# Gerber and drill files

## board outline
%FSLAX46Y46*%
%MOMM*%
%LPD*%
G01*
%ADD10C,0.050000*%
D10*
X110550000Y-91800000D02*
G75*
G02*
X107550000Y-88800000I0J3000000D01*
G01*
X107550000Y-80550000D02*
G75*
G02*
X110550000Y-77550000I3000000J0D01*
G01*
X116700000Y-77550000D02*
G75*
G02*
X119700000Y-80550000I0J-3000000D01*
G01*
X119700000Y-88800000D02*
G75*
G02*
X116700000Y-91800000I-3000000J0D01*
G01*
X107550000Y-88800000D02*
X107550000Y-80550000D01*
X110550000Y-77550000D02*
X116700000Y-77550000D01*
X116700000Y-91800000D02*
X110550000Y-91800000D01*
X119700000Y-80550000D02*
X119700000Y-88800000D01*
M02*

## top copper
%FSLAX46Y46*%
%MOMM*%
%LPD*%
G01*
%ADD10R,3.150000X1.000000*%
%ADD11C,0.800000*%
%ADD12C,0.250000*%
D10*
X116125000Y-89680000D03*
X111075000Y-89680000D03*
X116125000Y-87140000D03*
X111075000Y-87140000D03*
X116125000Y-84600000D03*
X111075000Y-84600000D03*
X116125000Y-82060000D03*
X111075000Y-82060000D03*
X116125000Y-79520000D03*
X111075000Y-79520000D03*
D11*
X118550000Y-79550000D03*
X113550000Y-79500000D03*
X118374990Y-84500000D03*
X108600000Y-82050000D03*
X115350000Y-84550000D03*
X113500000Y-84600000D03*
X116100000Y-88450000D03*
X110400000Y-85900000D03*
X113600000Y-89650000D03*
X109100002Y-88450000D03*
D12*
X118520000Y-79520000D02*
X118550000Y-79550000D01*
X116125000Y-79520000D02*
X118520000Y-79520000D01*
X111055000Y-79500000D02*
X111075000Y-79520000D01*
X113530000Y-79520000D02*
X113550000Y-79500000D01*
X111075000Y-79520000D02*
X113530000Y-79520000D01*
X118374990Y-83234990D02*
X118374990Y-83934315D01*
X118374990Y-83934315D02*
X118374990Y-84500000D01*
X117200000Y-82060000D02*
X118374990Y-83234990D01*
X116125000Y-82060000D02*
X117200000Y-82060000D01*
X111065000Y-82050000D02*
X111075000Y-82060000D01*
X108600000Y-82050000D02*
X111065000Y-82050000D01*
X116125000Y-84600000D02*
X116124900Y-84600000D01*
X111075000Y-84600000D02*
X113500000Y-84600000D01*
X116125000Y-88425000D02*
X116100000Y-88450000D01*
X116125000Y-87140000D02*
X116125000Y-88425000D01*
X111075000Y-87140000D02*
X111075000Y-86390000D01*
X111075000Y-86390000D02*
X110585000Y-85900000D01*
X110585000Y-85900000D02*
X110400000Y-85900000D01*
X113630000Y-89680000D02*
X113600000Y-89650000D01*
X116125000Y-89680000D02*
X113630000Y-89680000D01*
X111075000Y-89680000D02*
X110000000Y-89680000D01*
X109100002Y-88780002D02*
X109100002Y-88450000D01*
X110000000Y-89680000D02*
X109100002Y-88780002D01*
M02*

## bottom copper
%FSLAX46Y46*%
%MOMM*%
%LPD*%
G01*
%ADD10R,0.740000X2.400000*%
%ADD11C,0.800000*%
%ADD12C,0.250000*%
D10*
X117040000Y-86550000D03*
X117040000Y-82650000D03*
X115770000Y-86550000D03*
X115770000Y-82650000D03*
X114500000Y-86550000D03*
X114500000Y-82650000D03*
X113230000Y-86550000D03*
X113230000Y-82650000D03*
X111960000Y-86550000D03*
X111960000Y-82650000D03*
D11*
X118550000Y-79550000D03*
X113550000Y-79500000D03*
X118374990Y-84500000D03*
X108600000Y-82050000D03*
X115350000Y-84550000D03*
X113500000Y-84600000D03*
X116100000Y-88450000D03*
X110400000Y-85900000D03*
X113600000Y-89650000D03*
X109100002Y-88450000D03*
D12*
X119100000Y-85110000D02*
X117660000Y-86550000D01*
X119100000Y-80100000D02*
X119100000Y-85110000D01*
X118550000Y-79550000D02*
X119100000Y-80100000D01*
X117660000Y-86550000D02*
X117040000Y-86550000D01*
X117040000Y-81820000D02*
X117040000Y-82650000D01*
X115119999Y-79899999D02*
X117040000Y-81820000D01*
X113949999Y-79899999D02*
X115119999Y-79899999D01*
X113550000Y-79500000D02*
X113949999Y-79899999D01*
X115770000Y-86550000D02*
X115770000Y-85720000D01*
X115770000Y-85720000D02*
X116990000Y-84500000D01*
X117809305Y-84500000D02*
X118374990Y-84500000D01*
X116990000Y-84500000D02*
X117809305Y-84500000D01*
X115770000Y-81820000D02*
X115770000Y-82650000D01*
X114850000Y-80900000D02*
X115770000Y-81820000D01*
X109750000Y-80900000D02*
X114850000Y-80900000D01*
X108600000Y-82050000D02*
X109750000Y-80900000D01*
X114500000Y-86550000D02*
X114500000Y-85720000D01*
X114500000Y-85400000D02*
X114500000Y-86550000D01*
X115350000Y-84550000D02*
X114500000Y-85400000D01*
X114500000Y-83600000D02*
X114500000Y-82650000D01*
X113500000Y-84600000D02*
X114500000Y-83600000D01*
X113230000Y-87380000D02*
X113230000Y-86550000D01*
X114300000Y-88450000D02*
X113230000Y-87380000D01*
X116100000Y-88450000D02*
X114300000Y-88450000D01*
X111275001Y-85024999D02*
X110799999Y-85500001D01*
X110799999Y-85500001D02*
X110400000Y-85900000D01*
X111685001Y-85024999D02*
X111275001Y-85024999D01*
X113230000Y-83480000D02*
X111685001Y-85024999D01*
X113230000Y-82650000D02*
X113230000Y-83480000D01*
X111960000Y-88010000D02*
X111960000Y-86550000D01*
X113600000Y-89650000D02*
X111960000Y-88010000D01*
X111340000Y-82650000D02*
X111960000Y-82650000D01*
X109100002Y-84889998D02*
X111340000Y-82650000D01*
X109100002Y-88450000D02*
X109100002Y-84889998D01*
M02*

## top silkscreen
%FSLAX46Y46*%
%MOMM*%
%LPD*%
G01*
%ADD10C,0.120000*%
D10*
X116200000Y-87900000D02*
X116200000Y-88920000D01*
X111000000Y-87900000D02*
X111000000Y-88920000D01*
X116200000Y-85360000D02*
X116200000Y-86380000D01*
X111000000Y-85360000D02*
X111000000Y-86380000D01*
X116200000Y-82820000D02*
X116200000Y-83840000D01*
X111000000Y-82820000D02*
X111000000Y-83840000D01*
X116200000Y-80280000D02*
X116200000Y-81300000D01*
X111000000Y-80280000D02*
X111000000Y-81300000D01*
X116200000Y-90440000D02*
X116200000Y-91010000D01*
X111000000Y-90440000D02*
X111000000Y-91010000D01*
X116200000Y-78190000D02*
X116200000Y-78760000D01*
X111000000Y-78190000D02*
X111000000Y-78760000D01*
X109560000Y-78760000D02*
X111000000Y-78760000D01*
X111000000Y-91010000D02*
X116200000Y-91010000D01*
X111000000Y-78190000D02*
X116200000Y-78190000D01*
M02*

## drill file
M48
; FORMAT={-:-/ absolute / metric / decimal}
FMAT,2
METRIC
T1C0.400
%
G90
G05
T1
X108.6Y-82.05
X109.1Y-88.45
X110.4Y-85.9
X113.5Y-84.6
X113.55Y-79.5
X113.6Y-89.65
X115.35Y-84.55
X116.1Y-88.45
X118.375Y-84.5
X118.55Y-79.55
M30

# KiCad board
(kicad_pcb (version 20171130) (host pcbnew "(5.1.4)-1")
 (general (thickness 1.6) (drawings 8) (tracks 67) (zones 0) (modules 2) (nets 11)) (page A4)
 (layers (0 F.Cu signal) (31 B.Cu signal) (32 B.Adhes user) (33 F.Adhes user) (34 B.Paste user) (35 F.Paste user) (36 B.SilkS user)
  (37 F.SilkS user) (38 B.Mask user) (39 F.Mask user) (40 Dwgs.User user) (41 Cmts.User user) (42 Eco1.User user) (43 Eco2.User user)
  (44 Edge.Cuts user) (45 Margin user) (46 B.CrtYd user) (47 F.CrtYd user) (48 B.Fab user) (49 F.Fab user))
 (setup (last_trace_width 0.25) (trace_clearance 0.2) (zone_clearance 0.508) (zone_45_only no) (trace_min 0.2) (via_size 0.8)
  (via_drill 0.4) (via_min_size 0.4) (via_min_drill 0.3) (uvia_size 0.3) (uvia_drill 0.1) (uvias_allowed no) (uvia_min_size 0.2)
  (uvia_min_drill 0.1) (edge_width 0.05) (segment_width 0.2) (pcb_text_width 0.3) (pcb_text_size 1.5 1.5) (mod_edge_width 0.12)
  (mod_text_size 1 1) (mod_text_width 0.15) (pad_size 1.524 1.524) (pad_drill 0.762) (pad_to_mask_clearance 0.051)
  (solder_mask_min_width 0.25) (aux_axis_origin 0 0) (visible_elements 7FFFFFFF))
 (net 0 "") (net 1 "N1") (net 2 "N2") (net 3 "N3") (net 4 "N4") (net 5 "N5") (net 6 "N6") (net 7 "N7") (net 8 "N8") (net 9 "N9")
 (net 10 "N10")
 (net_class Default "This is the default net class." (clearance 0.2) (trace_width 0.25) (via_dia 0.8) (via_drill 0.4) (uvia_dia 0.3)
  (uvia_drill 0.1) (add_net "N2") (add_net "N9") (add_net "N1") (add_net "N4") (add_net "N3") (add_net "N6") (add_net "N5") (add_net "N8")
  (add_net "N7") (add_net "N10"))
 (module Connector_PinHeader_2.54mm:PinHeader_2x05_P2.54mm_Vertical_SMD (layer F.Cu) (at 113.6 84.6)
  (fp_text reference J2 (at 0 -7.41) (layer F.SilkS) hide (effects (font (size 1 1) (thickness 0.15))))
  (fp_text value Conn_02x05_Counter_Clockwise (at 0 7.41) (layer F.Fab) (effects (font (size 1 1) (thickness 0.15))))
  (fp_line (start 2.6 3.3) (end 2.6 4.32) (layer F.SilkS) (width 0.12))
  (fp_line (start -2.6 3.3) (end -2.6 4.32) (layer F.SilkS) (width 0.12))
  (fp_line (start 2.6 0.76) (end 2.6 1.78) (layer F.SilkS) (width 0.12))
  (fp_line (start -2.6 0.76) (end -2.6 1.78) (layer F.SilkS) (width 0.12))
  (fp_line (start 2.6 -1.78) (end 2.6 -0.76) (layer F.SilkS) (width 0.12))
  (fp_line (start -2.6 -1.78) (end -2.6 -0.76) (layer F.SilkS) (width 0.12))
  (fp_line (start 2.6 -4.32) (end 2.6 -3.3) (layer F.SilkS) (width 0.12))
  (fp_line (start -2.6 -4.32) (end -2.6 -3.3) (layer F.SilkS) (width 0.12))
  (fp_line (start 2.6 5.84) (end 2.6 6.41) (layer F.SilkS) (width 0.12))
  (fp_line (start -2.6 5.84) (end -2.6 6.41) (layer F.SilkS) (width 0.12))
  (fp_line (start 2.6 -6.41) (end 2.6 -5.84) (layer F.SilkS) (width 0.12))
  (fp_line (start -2.6 -6.41) (end -2.6 -5.84) (layer F.SilkS) (width 0.12))
  (fp_line (start -4.04 -5.84) (end -2.6 -5.84) (layer F.SilkS) (width 0.12))
  (fp_line (start -2.6 6.41) (end 2.6 6.41) (layer F.SilkS) (width 0.12))
  (fp_line (start -2.6 -6.41) (end 2.6 -6.41) (layer F.SilkS) (width 0.12))
  (pad 10 smd rect (at 2.525 5.08) (size 3.15 1) (layers F.Cu F.Paste F.Mask) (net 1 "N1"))
  (pad 9 smd rect (at -2.525 5.08) (size 3.15 1) (layers F.Cu F.Paste F.Mask) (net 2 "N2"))
  (pad 8 smd rect (at 2.525 2.54) (size 3.15 1) (layers F.Cu F.Paste F.Mask) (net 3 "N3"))
  (pad 7 smd rect (at -2.525 2.54) (size 3.15 1) (layers F.Cu F.Paste F.Mask) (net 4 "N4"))
  (pad 6 smd rect (at 2.525 0) (size 3.15 1) (layers F.Cu F.Paste F.Mask) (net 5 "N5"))
  (pad 5 smd rect (at -2.525 0) (size 3.15 1) (layers F.Cu F.Paste F.Mask) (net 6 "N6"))
  (pad 4 smd rect (at 2.525 -2.54) (size 3.15 1) (layers F.Cu F.Paste F.Mask) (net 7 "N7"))
  (pad 3 smd rect (at -2.525 -2.54) (size 3.15 1) (layers F.Cu F.Paste F.Mask) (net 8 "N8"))
  (pad 2 smd rect (at 2.525 -5.08) (size 3.15 1) (layers F.Cu F.Paste F.Mask) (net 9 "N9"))
  (pad 1 smd rect (at -2.525 -5.08) (size 3.15 1) (layers F.Cu F.Paste F.Mask) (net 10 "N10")))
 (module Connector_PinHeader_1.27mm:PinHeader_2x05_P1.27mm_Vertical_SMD (layer B.Cu) (at 114.5 84.6 270)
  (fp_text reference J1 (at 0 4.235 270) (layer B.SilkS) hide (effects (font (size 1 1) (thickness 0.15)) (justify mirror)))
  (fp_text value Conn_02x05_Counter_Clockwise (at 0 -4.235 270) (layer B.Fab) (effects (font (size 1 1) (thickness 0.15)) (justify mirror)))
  (pad 10 smd rect (at 1.95 -2.54 270) (size 2.4 0.74) (layers B.Cu B.Paste B.Mask) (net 9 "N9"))
  (pad 9 smd rect (at -1.95 -2.54 270) (size 2.4 0.74) (layers B.Cu B.Paste B.Mask) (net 10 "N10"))
  (pad 8 smd rect (at 1.95 -1.27 270) (size 2.4 0.74) (layers B.Cu B.Paste B.Mask) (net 7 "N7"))
  (pad 7 smd rect (at -1.95 -1.27 270) (size 2.4 0.74) (layers B.Cu B.Paste B.Mask) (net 8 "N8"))
  (pad 6 smd rect (at 1.95 0 270) (size 2.4 0.74) (layers B.Cu B.Paste B.Mask) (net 5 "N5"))
  (pad 5 smd rect (at -1.95 0 270) (size 2.4 0.74) (layers B.Cu B.Paste B.Mask) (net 6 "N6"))
  (pad 4 smd rect (at 1.95 1.27 270) (size 2.4 0.74) (layers B.Cu B.Paste B.Mask) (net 3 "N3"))
  (pad 3 smd rect (at -1.95 1.27 270) (size 2.4 0.74) (layers B.Cu B.Paste B.Mask) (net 4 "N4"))
  (pad 2 smd rect (at 1.95 2.54 270) (size 2.4 0.74) (layers B.Cu B.Paste B.Mask) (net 1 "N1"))
  (pad 1 smd rect (at -1.95 2.54 270) (size 2.4 0.74) (layers B.Cu B.Paste B.Mask) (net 2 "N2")))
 (gr_arc (start 110.55 88.8) (end 110.55 91.8) (angle 90) (layer Edge.Cuts) (width 0.05))
 (gr_arc (start 110.55 80.55) (end 107.55 80.55) (angle 90) (layer Edge.Cuts) (width 0.05))
 (gr_arc (start 116.7 80.55) (end 116.7 77.55) (angle 90) (layer Edge.Cuts) (width 0.05))
 (gr_arc (start 116.7 88.8) (end 119.7 88.8) (angle 90) (layer Edge.Cuts) (width 0.05))
 (gr_line (start 107.55 88.8) (end 107.55 80.55) (layer Edge.Cuts) (width 0.05))
 (gr_line (start 110.55 77.55) (end 116.7 77.55) (layer Edge.Cuts) (width 0.05))
 (gr_line (start 116.7 91.8) (end 110.55 91.8) (layer Edge.Cuts) (width 0.05))
 (gr_line (start 119.7 80.55) (end 119.7 88.8) (layer Edge.Cuts) (width 0.05))
 (via (at 118.55 79.55) (size 0.8) (drill 0.4) (layers F.Cu B.Cu) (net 9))
 (segment (start 118.52 79.52) (end 118.55 79.55) (width 0.25) (layer F.Cu) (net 9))
 (segment (start 116.125 79.52) (end 118.52 79.52) (width 0.25) (layer F.Cu) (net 9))
 (segment (start 119.1 85.11) (end 117.66 86.55) (width 0.25) (layer B.Cu) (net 9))
 (segment (start 119.1 80.1) (end 119.1 85.11) (width 0.25) (layer B.Cu) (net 9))
 (segment (start 118.55 79.55) (end 119.1 80.1) (width 0.25) (layer B.Cu) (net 9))
 (segment (start 117.66 86.55) (end 117.04 86.55) (width 0.25) (layer B.Cu) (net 9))
 (via (at 113.55 79.5) (size 0.8) (drill 0.4) (layers F.Cu B.Cu) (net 10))
 (segment (start 111.055 79.5) (end 111.075 79.52) (width 0.25) (layer F.Cu) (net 10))
 (segment (start 113.53 79.52) (end 113.55 79.5) (width 0.25) (layer F.Cu) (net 10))
 (segment (start 111.075 79.52) (end 113.53 79.52) (width 0.25) (layer F.Cu) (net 10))
 (segment (start 117.04 81.82) (end 117.04 82.65) (width 0.25) (layer B.Cu) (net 10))
 (segment (start 115.119999 79.899999) (end 117.04 81.82) (width 0.25) (layer B.Cu) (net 10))
 (segment (start 113.949999 79.899999) (end 115.119999 79.899999) (width 0.25) (layer B.Cu) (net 10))
 (segment (start 113.55 79.5) (end 113.949999 79.899999) (width 0.25) (layer B.Cu) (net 10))
 (via (at 118.37499 84.5) (size 0.8) (drill 0.4) (layers F.Cu B.Cu) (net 7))
 (segment (start 115.77 86.55) (end 115.77 85.72) (width 0.25) (layer B.Cu) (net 7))
 (segment (start 115.77 85.72) (end 116.99 84.5) (width 0.25) (layer B.Cu) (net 7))
 (segment (start 118.37499 83.23499) (end 118.37499 83.934315) (width 0.25) (layer F.Cu) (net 7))
 (segment (start 118.37499 83.934315) (end 118.37499 84.5) (width 0.25) (layer F.Cu) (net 7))
 (segment (start 117.2 82.06) (end 118.37499 83.23499) (width 0.25) (layer F.Cu) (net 7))
 (segment (start 117.809305 84.5) (end 118.37499 84.5) (width 0.25) (layer B.Cu) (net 7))
 (segment (start 116.125 82.06) (end 117.2 82.06) (width 0.25) (layer F.Cu) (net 7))
 (segment (start 116.99 84.5) (end 117.809305 84.5) (width 0.25) (layer B.Cu) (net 7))
 (via (at 108.6 82.05) (size 0.8) (drill 0.4) (layers F.Cu B.Cu) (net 8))
 (segment (start 111.065 82.05) (end 111.075 82.06) (width 0.25) (layer F.Cu) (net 8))
 (segment (start 108.6 82.05) (end 111.065 82.05) (width 0.25) (layer F.Cu) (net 8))
 (segment (start 115.77 81.82) (end 115.77 82.65) (width 0.25) (layer B.Cu) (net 8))
 (segment (start 114.85 80.9) (end 115.77 81.82) (width 0.25) (layer B.Cu) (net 8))
 (segment (start 109.75 80.9) (end 114.85 80.9) (width 0.25) (layer B.Cu) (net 8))
 (segment (start 108.6 82.05) (end 109.75 80.9) (width 0.25) (layer B.Cu) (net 8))
 (via (at 115.35 84.55) (size 0.8) (drill 0.4) (layers F.Cu B.Cu) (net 5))
 (segment (start 116.125 84.6) (end 116.1249 84.6) (width 0.25) (layer F.Cu) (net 5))
 (segment (start 114.5 86.55) (end 114.5 85.72) (width 0.25) (layer B.Cu) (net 5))
 (segment (start 114.5 85.4) (end 114.5 86.55) (width 0.25) (layer B.Cu) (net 5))
 (segment (start 115.35 84.55) (end 114.5 85.4) (width 0.25) (layer B.Cu) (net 5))
 (via (at 113.5 84.6) (size 0.8) (drill 0.4) (layers F.Cu B.Cu) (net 6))
 (segment (start 111.075 84.6) (end 113.5 84.6) (width 0.25) (layer F.Cu) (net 6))
 (segment (start 114.5 83.6) (end 114.5 82.65) (width 0.25) (layer B.Cu) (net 6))
 (segment (start 113.5 84.6) (end 114.5 83.6) (width 0.25) (layer B.Cu) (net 6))
 (via (at 116.1 88.45) (size 0.8) (drill 0.4) (layers F.Cu B.Cu) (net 3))
 (segment (start 116.125 88.425) (end 116.1 88.45) (width 0.25) (layer F.Cu) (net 3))
 (segment (start 116.125 87.14) (end 116.125 88.425) (width 0.25) (layer F.Cu) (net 3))
 (segment (start 113.23 87.38) (end 113.23 86.55) (width 0.25) (layer B.Cu) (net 3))
 (segment (start 114.3 88.45) (end 113.23 87.38) (width 0.25) (layer B.Cu) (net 3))
 (segment (start 116.1 88.45) (end 114.3 88.45) (width 0.25) (layer B.Cu) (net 3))
 (via (at 110.4 85.9) (size 0.8) (drill 0.4) (layers F.Cu B.Cu) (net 4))
 (segment (start 111.075 87.14) (end 111.075 86.39) (width 0.25) (layer F.Cu) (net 4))
 (segment (start 111.075 86.39) (end 110.585 85.9) (width 0.25) (layer F.Cu) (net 4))
 (segment (start 111.275001 85.024999) (end 110.799999 85.500001) (width 0.25) (layer B.Cu) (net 4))
 (segment (start 110.799999 85.500001) (end 110.4 85.9) (width 0.25) (layer B.Cu) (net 4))
 (segment (start 111.685001 85.024999) (end 111.275001 85.024999) (width 0.25) (layer B.Cu) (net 4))
 (segment (start 113.23 83.48) (end 111.685001 85.024999) (width 0.25) (layer B.Cu) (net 4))
 (segment (start 113.23 82.65) (end 113.23 83.48) (width 0.25) (layer B.Cu) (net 4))
 (segment (start 110.585 85.9) (end 110.4 85.9) (width 0.25) (layer F.Cu) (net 4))
 (via (at 113.6 89.65) (size 0.8) (drill 0.4) (layers F.Cu B.Cu) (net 1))
 (segment (start 113.63 89.68) (end 113.6 89.65) (width 0.25) (layer F.Cu) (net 1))
 (segment (start 116.125 89.68) (end 113.63 89.68) (width 0.25) (layer F.Cu) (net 1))
 (segment (start 111.96 88.01) (end 111.96 86.55) (width 0.25) (layer B.Cu) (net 1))
 (segment (start 113.6 89.65) (end 111.96 88.01) (width 0.25) (layer B.Cu) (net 1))
 (via (at 109.100002 88.45) (size 0.8) (drill 0.4) (layers F.Cu B.Cu) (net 2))
 (segment (start 111.075 89.68) (end 110 89.68) (width 0.25) (layer F.Cu) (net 2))
 (segment (start 109.100002 88.780002) (end 109.100002 88.45) (width 0.25) (layer F.Cu) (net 2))
 (segment (start 110 89.68) (end 109.100002 88.780002) (width 0.25) (layer F.Cu) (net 2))
 (segment (start 111.34 82.65) (end 111.96 82.65) (width 0.25) (layer B.Cu) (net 2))
 (segment (start 109.100002 84.889998) (end 111.34 82.65) (width 0.25) (layer B.Cu) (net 2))
 (segment (start 109.100002 88.45) (end 109.100002 84.889998) (width 0.25) (layer B.Cu) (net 2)))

